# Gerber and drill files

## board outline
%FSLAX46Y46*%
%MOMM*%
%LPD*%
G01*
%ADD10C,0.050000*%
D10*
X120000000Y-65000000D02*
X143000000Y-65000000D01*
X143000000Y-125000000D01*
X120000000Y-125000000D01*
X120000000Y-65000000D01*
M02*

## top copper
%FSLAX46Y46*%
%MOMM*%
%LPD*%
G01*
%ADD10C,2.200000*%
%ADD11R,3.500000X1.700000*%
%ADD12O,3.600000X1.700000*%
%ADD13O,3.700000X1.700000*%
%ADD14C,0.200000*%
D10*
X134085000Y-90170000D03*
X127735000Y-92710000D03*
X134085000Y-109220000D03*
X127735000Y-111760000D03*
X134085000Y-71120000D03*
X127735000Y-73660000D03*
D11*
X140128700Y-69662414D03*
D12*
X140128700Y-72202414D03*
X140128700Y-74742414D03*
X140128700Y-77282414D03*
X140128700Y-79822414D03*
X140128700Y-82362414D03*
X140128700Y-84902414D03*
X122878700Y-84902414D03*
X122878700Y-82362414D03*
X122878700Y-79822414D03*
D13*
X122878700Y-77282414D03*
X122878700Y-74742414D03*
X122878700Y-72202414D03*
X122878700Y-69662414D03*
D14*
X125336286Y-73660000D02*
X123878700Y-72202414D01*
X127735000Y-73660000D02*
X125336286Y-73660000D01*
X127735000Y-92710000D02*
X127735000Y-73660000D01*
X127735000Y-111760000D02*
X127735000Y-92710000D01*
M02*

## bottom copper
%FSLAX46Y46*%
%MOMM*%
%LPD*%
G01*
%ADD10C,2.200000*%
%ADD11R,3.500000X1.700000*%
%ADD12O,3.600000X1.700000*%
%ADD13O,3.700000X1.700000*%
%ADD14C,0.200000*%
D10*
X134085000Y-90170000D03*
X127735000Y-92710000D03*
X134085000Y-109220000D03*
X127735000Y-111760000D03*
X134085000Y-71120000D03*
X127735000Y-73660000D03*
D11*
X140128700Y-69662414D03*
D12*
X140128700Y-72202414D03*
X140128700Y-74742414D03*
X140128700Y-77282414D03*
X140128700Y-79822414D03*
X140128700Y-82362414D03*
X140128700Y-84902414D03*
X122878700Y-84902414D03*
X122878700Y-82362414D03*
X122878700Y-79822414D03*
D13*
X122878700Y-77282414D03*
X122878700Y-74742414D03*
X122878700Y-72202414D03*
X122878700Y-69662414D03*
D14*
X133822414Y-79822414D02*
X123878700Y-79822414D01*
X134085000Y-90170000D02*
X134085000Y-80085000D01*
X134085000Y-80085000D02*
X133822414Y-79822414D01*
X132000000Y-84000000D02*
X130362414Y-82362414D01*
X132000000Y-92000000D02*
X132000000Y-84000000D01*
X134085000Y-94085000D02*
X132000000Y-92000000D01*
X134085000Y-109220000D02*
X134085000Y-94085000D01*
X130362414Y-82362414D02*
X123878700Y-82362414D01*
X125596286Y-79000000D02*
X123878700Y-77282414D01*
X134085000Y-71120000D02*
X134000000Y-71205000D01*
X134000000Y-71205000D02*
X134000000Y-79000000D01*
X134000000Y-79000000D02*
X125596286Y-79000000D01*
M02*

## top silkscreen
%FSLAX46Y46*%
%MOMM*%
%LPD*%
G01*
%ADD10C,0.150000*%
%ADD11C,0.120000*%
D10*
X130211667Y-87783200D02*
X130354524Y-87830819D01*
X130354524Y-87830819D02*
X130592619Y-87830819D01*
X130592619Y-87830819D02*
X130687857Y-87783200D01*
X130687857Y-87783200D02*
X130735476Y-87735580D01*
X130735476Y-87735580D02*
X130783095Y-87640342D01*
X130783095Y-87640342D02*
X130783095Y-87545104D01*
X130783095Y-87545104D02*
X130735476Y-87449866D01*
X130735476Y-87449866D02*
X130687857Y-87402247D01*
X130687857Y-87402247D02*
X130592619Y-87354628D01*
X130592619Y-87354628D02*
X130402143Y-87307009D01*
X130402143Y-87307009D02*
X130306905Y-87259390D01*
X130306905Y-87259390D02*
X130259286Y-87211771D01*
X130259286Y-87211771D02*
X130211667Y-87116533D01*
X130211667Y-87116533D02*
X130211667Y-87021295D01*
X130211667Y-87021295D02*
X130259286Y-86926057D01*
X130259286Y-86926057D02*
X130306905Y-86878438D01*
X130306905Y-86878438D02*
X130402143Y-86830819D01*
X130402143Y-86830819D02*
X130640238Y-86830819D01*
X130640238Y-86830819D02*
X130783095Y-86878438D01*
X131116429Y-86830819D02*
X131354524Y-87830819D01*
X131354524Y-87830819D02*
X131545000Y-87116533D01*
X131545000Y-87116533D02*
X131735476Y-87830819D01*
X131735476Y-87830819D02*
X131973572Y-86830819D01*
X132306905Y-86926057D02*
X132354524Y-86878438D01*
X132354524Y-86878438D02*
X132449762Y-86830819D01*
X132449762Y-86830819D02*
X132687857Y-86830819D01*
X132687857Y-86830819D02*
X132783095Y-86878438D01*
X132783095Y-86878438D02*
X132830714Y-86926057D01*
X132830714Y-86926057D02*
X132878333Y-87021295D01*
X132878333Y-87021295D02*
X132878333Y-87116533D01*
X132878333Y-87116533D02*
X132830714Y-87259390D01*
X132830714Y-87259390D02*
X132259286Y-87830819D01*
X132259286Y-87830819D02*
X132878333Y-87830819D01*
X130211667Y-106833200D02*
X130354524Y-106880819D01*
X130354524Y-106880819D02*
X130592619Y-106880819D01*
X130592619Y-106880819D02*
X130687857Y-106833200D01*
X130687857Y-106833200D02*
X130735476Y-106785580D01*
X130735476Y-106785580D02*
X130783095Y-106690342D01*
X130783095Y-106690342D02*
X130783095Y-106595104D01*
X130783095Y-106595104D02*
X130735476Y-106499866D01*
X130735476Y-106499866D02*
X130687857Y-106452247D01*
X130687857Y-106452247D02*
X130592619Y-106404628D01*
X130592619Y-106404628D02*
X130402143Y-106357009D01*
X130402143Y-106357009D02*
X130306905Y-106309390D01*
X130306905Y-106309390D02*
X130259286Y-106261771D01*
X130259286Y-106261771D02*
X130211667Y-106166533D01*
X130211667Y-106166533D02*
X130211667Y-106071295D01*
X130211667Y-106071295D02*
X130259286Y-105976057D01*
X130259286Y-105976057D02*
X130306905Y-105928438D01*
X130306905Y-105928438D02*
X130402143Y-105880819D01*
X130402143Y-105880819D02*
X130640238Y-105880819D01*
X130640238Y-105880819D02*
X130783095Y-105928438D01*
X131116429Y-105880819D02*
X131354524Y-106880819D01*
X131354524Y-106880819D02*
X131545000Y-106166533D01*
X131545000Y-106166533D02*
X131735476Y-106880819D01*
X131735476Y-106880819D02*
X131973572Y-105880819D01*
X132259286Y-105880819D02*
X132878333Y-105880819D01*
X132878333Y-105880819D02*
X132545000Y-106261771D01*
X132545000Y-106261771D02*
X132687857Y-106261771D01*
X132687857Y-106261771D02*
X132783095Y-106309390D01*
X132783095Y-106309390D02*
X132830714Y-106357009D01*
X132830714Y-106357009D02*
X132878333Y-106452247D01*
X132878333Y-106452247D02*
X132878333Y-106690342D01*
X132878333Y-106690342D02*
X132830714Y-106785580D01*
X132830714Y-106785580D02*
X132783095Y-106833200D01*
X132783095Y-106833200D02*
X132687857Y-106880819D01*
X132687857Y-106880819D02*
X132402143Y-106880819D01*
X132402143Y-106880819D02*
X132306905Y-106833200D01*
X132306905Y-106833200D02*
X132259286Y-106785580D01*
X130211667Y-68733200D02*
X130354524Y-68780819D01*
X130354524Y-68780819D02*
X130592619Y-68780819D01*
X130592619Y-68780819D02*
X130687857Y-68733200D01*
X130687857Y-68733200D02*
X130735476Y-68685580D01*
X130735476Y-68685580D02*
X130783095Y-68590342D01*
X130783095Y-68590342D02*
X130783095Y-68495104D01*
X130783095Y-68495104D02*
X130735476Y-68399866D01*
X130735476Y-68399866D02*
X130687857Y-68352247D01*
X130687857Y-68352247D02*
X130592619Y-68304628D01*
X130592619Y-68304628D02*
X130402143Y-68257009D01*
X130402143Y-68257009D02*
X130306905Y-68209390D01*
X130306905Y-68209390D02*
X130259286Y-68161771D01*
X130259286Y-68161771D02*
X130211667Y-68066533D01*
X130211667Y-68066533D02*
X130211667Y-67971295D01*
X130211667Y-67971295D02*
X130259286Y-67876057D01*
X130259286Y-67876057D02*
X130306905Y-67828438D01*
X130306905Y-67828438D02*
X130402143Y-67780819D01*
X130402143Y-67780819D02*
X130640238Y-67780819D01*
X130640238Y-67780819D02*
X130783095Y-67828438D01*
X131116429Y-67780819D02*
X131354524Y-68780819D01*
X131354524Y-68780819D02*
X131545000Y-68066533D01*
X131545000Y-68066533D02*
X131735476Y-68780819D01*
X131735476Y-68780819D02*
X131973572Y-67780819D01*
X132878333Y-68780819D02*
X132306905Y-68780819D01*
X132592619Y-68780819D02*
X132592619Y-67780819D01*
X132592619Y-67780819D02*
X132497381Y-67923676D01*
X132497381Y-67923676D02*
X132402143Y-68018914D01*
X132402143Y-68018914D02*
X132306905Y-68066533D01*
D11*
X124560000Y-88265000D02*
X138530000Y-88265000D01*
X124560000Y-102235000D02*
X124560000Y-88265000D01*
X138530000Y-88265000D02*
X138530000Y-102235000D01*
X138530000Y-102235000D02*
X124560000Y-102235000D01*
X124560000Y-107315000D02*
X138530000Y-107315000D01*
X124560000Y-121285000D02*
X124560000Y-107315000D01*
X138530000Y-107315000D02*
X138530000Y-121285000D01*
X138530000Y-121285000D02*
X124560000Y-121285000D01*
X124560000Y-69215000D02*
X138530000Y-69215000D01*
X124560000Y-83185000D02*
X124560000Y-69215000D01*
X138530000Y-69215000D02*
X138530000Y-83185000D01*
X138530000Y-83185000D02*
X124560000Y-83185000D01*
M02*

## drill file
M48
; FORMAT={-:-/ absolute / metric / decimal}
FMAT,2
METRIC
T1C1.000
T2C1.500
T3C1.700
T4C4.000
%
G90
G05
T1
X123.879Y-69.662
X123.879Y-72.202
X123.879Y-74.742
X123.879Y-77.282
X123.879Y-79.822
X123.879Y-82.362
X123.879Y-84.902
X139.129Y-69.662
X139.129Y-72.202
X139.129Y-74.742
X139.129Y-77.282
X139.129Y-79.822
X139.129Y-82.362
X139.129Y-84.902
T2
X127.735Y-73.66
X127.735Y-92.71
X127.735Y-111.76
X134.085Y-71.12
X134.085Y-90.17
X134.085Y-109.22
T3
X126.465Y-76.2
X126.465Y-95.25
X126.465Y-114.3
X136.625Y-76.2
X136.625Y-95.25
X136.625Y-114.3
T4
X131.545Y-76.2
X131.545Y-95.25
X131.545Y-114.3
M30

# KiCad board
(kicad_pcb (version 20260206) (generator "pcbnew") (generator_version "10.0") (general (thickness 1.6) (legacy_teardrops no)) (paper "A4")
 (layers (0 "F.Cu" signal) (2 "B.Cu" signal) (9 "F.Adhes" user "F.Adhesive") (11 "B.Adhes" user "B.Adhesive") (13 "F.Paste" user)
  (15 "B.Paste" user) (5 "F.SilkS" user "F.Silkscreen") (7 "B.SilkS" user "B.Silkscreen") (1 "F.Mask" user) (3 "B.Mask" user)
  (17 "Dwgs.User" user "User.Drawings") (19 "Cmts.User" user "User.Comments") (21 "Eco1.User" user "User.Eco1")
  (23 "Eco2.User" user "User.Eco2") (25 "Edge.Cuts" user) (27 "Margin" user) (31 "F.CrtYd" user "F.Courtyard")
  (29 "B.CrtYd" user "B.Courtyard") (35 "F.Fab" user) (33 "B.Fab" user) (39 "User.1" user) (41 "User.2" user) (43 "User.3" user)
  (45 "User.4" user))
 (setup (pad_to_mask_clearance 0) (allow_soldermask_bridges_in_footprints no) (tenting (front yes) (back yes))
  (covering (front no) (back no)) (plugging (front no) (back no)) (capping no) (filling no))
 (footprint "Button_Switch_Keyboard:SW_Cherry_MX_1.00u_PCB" (layer "F.Cu") (at 134.085 90.17)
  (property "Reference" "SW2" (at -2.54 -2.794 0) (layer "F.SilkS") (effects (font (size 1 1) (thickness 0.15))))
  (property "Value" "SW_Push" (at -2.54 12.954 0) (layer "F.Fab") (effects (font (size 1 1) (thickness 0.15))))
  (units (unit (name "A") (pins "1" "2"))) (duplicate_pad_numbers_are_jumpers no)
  (fp_line (start -9.525 -1.905) (end 4.445 -1.905) (stroke (width 0.12) (type solid)) (layer "F.SilkS"))
  (fp_line (start -9.525 12.065) (end -9.525 -1.905) (stroke (width 0.12) (type solid)) (layer "F.SilkS"))
  (fp_line (start 4.445 -1.905) (end 4.445 12.065) (stroke (width 0.12) (type solid)) (layer "F.SilkS"))
  (fp_line (start 4.445 12.065) (end -9.525 12.065) (stroke (width 0.12) (type solid)) (layer "F.SilkS"))
  (pad "" np_thru_hole circle (at -7.62 5.08) (size 1.7 1.7) (drill 1.7) (layers "*.Cu" "*.Mask"))
  (pad "" np_thru_hole circle (at -2.54 5.08) (size 4 4) (drill 4) (layers "*.Cu" "*.Mask"))
  (pad "" np_thru_hole circle (at 2.54 5.08) (size 1.7 1.7) (drill 1.7) (layers "*.Cu" "*.Mask"))
  (pad "1" thru_hole circle (at 0 0) (size 2.2 2.2) (drill 1.5) (layers "*.Cu" "*.Mask") (remove_unused_layers no)
   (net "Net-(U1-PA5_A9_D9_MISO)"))
  (pad "2" thru_hole circle (at -6.35 2.54) (size 2.2 2.2) (drill 1.5) (layers "*.Cu" "*.Mask") (remove_unused_layers no) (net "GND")))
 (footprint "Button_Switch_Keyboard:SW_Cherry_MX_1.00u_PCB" (layer "F.Cu") (at 134.085 109.22)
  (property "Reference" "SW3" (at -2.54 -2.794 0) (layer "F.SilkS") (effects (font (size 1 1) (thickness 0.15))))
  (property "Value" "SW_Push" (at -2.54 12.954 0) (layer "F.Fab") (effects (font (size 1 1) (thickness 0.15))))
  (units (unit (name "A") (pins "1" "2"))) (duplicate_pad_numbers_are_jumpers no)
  (fp_line (start -9.525 -1.905) (end 4.445 -1.905) (stroke (width 0.12) (type solid)) (layer "F.SilkS"))
  (fp_line (start -9.525 12.065) (end -9.525 -1.905) (stroke (width 0.12) (type solid)) (layer "F.SilkS"))
  (fp_line (start 4.445 -1.905) (end 4.445 12.065) (stroke (width 0.12) (type solid)) (layer "F.SilkS"))
  (fp_line (start 4.445 12.065) (end -9.525 12.065) (stroke (width 0.12) (type solid)) (layer "F.SilkS"))
  (pad "" np_thru_hole circle (at -7.62 5.08) (size 1.7 1.7) (drill 1.7) (layers "*.Cu" "*.Mask"))
  (pad "" np_thru_hole circle (at -2.54 5.08) (size 4 4) (drill 4) (layers "*.Cu" "*.Mask"))
  (pad "" np_thru_hole circle (at 2.54 5.08) (size 1.7 1.7) (drill 1.7) (layers "*.Cu" "*.Mask"))
  (pad "1" thru_hole circle (at 0 0) (size 2.2 2.2) (drill 1.5) (layers "*.Cu" "*.Mask") (remove_unused_layers no)
   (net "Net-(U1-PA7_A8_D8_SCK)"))
  (pad "2" thru_hole circle (at -6.35 2.54) (size 2.2 2.2) (drill 1.5) (layers "*.Cu" "*.Mask") (remove_unused_layers no) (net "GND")))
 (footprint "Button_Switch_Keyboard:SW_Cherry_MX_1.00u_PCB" (layer "F.Cu") (at 134.085 71.12)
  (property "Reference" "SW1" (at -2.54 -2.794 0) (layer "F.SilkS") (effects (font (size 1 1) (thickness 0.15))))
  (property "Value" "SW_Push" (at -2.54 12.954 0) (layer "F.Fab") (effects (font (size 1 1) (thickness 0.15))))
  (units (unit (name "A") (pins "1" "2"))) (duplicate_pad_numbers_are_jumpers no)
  (fp_line (start -9.525 -1.905) (end 4.445 -1.905) (stroke (width 0.12) (type solid)) (layer "F.SilkS"))
  (fp_line (start -9.525 12.065) (end -9.525 -1.905) (stroke (width 0.12) (type solid)) (layer "F.SilkS"))
  (fp_line (start 4.445 -1.905) (end 4.445 12.065) (stroke (width 0.12) (type solid)) (layer "F.SilkS"))
  (fp_line (start 4.445 12.065) (end -9.525 12.065) (stroke (width 0.12) (type solid)) (layer "F.SilkS"))
  (pad "" np_thru_hole circle (at -7.62 5.08) (size 1.7 1.7) (drill 1.7) (layers "*.Cu" "*.Mask"))
  (pad "" np_thru_hole circle (at -2.54 5.08) (size 4 4) (drill 4) (layers "*.Cu" "*.Mask"))
  (pad "" np_thru_hole circle (at 2.54 5.08) (size 1.7 1.7) (drill 1.7) (layers "*.Cu" "*.Mask"))
  (pad "1" thru_hole circle (at 0 0) (size 2.2 2.2) (drill 1.5) (layers "*.Cu" "*.Mask") (remove_unused_layers no)
   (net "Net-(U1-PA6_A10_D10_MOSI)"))
  (pad "2" thru_hole circle (at -6.35 2.54) (size 2.2 2.2) (drill 1.5) (layers "*.Cu" "*.Mask") (remove_unused_layers no) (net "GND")))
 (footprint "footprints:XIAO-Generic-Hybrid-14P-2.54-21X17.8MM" (layer "B.Cu") (at 131.5037 77.282414 180)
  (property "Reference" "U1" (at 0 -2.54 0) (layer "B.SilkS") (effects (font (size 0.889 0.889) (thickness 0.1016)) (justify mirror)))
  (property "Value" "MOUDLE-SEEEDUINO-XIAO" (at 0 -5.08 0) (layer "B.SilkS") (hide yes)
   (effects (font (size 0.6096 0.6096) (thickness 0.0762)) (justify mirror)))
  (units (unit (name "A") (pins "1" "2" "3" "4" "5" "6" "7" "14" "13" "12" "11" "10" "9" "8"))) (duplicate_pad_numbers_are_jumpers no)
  (pad "1" thru_hole rect (at -7.625 7.62 180) (size 3.5 1.7) (drill 1 (offset -1 0)) (layers "*.Cu" "*.Mask") (remove_unused_layers no)
   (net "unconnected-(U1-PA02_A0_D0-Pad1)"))
  (pad "2" thru_hole oval (at -7.625 5.08 180) (size 3.6 1.7) (drill 1 (offset -1 0)) (layers "*.Cu" "*.Mask") (remove_unused_layers no)
   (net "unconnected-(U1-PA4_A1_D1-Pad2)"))
  (pad "3" thru_hole oval (at -7.625 2.54 180) (size 3.6 1.7) (drill 1 (offset -1 0)) (layers "*.Cu" "*.Mask") (remove_unused_layers no)
   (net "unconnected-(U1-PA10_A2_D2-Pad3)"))
  (pad "4" thru_hole oval (at -7.625 0 180) (size 3.6 1.7) (drill 1 (offset -1 0)) (layers "*.Cu" "*.Mask") (remove_unused_layers no)
   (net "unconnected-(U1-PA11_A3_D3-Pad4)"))
  (pad "5" thru_hole oval (at -7.625 -2.54 180) (size 3.6 1.7) (drill 1 (offset -1 0)) (layers "*.Cu" "*.Mask") (remove_unused_layers no)
   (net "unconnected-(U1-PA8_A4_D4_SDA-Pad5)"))
  (pad "6" thru_hole oval (at -7.625 -5.08) (size 3.6 1.7) (drill 1 (offset 1 0)) (layers "*.Cu" "*.Mask") (remove_unused_layers no)
   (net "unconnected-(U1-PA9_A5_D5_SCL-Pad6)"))
  (pad "7" thru_hole oval (at -7.625 -7.62 180) (size 3.6 1.7) (drill 1 (offset -1 0)) (layers "*.Cu" "*.Mask") (remove_unused_layers no)
   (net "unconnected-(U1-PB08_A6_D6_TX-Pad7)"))
  (pad "8" thru_hole oval (at 7.625 -7.62 180) (size 3.6 1.7) (drill 1 (offset 1 0)) (layers "*.Cu" "*.Mask") (remove_unused_layers no)
   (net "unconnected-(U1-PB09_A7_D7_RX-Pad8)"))
  (pad "9" thru_hole oval (at 7.625 -5.08 180) (size 3.6 1.7) (drill 1 (offset 1 0)) (layers "*.Cu" "*.Mask") (remove_unused_layers no)
   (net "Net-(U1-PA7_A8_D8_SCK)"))
  (pad "10" thru_hole oval (at 7.625 -2.54 180) (size 3.6 1.7) (drill 1 (offset 1 0)) (layers "*.Cu" "*.Mask") (remove_unused_layers no)
   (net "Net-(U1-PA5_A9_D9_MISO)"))
  (pad "11" thru_hole oval (at 7.625 0 180) (size 3.7 1.7) (drill 1 (offset 1 0)) (layers "*.Cu" "*.Mask") (remove_unused_layers no)
   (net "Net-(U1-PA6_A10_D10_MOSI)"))
  (pad "12" thru_hole oval (at 7.625 2.54 180) (size 3.7 1.7) (drill 1 (offset 1 0)) (layers "*.Cu" "*.Mask") (remove_unused_layers no)
   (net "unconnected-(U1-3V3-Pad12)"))
  (pad "13" thru_hole oval (at 7.625 5.08 180) (size 3.7 1.7) (drill 1 (offset 1 0)) (layers "*.Cu" "*.Mask") (remove_unused_layers no)
   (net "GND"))
  (pad "14" thru_hole oval (at 7.625 7.62 180) (size 3.7 1.7) (drill 1 (offset 1 0)) (layers "*.Cu" "*.Mask") (remove_unused_layers no)
   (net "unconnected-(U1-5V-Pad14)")))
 (gr_rect (start 120 65) (end 143 125) (stroke (width 0.05) (type default)) (fill no) (layer "Edge.Cuts"))
 (segment (start 133.822414 79.822414) (end 123.8787 79.822414) (width 0.2) (layer "B.Cu") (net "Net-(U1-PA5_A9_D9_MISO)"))
 (segment (start 134.085 90.17) (end 134.085 80.085) (width 0.2) (layer "B.Cu") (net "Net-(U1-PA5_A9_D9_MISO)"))
 (segment (start 134.085 80.085) (end 133.822414 79.822414) (width 0.2) (layer "B.Cu") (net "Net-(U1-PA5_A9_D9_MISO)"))
 (segment (start 125.336286 73.66) (end 123.8787 72.202414) (width 0.2) (layer "F.Cu") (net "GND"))
 (segment (start 127.735 73.66) (end 125.336286 73.66) (width 0.2) (layer "F.Cu") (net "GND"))
 (segment (start 127.735 92.71) (end 127.735 73.66) (width 0.2) (layer "F.Cu") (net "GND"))
 (segment (start 127.735 111.76) (end 127.735 92.71) (width 0.2) (layer "F.Cu") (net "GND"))
 (segment (start 132 84) (end 130.362414 82.362414) (width 0.2) (layer "B.Cu") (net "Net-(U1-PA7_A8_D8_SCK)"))
 (segment (start 132 92) (end 132 84) (width 0.2) (layer "B.Cu") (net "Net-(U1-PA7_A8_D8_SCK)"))
 (segment (start 134.085 94.085) (end 132 92) (width 0.2) (layer "B.Cu") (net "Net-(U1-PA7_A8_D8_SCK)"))
 (segment (start 134.085 109.22) (end 134.085 94.085) (width 0.2) (layer "B.Cu") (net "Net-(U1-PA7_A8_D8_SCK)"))
 (segment (start 130.362414 82.362414) (end 123.8787 82.362414) (width 0.2) (layer "B.Cu") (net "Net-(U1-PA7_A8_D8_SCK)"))
 (segment (start 125.596286 79) (end 123.8787 77.282414) (width 0.2) (layer "B.Cu") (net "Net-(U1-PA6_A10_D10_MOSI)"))
 (segment (start 134.085 71.12) (end 134 71.205) (width 0.2) (layer "B.Cu") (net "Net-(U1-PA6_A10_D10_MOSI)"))
 (segment (start 134 71.205) (end 134 79) (width 0.2) (layer "B.Cu") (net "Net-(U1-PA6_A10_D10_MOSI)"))
 (segment (start 134 79) (end 125.596286 79) (width 0.2) (layer "B.Cu") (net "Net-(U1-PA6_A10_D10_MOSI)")))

